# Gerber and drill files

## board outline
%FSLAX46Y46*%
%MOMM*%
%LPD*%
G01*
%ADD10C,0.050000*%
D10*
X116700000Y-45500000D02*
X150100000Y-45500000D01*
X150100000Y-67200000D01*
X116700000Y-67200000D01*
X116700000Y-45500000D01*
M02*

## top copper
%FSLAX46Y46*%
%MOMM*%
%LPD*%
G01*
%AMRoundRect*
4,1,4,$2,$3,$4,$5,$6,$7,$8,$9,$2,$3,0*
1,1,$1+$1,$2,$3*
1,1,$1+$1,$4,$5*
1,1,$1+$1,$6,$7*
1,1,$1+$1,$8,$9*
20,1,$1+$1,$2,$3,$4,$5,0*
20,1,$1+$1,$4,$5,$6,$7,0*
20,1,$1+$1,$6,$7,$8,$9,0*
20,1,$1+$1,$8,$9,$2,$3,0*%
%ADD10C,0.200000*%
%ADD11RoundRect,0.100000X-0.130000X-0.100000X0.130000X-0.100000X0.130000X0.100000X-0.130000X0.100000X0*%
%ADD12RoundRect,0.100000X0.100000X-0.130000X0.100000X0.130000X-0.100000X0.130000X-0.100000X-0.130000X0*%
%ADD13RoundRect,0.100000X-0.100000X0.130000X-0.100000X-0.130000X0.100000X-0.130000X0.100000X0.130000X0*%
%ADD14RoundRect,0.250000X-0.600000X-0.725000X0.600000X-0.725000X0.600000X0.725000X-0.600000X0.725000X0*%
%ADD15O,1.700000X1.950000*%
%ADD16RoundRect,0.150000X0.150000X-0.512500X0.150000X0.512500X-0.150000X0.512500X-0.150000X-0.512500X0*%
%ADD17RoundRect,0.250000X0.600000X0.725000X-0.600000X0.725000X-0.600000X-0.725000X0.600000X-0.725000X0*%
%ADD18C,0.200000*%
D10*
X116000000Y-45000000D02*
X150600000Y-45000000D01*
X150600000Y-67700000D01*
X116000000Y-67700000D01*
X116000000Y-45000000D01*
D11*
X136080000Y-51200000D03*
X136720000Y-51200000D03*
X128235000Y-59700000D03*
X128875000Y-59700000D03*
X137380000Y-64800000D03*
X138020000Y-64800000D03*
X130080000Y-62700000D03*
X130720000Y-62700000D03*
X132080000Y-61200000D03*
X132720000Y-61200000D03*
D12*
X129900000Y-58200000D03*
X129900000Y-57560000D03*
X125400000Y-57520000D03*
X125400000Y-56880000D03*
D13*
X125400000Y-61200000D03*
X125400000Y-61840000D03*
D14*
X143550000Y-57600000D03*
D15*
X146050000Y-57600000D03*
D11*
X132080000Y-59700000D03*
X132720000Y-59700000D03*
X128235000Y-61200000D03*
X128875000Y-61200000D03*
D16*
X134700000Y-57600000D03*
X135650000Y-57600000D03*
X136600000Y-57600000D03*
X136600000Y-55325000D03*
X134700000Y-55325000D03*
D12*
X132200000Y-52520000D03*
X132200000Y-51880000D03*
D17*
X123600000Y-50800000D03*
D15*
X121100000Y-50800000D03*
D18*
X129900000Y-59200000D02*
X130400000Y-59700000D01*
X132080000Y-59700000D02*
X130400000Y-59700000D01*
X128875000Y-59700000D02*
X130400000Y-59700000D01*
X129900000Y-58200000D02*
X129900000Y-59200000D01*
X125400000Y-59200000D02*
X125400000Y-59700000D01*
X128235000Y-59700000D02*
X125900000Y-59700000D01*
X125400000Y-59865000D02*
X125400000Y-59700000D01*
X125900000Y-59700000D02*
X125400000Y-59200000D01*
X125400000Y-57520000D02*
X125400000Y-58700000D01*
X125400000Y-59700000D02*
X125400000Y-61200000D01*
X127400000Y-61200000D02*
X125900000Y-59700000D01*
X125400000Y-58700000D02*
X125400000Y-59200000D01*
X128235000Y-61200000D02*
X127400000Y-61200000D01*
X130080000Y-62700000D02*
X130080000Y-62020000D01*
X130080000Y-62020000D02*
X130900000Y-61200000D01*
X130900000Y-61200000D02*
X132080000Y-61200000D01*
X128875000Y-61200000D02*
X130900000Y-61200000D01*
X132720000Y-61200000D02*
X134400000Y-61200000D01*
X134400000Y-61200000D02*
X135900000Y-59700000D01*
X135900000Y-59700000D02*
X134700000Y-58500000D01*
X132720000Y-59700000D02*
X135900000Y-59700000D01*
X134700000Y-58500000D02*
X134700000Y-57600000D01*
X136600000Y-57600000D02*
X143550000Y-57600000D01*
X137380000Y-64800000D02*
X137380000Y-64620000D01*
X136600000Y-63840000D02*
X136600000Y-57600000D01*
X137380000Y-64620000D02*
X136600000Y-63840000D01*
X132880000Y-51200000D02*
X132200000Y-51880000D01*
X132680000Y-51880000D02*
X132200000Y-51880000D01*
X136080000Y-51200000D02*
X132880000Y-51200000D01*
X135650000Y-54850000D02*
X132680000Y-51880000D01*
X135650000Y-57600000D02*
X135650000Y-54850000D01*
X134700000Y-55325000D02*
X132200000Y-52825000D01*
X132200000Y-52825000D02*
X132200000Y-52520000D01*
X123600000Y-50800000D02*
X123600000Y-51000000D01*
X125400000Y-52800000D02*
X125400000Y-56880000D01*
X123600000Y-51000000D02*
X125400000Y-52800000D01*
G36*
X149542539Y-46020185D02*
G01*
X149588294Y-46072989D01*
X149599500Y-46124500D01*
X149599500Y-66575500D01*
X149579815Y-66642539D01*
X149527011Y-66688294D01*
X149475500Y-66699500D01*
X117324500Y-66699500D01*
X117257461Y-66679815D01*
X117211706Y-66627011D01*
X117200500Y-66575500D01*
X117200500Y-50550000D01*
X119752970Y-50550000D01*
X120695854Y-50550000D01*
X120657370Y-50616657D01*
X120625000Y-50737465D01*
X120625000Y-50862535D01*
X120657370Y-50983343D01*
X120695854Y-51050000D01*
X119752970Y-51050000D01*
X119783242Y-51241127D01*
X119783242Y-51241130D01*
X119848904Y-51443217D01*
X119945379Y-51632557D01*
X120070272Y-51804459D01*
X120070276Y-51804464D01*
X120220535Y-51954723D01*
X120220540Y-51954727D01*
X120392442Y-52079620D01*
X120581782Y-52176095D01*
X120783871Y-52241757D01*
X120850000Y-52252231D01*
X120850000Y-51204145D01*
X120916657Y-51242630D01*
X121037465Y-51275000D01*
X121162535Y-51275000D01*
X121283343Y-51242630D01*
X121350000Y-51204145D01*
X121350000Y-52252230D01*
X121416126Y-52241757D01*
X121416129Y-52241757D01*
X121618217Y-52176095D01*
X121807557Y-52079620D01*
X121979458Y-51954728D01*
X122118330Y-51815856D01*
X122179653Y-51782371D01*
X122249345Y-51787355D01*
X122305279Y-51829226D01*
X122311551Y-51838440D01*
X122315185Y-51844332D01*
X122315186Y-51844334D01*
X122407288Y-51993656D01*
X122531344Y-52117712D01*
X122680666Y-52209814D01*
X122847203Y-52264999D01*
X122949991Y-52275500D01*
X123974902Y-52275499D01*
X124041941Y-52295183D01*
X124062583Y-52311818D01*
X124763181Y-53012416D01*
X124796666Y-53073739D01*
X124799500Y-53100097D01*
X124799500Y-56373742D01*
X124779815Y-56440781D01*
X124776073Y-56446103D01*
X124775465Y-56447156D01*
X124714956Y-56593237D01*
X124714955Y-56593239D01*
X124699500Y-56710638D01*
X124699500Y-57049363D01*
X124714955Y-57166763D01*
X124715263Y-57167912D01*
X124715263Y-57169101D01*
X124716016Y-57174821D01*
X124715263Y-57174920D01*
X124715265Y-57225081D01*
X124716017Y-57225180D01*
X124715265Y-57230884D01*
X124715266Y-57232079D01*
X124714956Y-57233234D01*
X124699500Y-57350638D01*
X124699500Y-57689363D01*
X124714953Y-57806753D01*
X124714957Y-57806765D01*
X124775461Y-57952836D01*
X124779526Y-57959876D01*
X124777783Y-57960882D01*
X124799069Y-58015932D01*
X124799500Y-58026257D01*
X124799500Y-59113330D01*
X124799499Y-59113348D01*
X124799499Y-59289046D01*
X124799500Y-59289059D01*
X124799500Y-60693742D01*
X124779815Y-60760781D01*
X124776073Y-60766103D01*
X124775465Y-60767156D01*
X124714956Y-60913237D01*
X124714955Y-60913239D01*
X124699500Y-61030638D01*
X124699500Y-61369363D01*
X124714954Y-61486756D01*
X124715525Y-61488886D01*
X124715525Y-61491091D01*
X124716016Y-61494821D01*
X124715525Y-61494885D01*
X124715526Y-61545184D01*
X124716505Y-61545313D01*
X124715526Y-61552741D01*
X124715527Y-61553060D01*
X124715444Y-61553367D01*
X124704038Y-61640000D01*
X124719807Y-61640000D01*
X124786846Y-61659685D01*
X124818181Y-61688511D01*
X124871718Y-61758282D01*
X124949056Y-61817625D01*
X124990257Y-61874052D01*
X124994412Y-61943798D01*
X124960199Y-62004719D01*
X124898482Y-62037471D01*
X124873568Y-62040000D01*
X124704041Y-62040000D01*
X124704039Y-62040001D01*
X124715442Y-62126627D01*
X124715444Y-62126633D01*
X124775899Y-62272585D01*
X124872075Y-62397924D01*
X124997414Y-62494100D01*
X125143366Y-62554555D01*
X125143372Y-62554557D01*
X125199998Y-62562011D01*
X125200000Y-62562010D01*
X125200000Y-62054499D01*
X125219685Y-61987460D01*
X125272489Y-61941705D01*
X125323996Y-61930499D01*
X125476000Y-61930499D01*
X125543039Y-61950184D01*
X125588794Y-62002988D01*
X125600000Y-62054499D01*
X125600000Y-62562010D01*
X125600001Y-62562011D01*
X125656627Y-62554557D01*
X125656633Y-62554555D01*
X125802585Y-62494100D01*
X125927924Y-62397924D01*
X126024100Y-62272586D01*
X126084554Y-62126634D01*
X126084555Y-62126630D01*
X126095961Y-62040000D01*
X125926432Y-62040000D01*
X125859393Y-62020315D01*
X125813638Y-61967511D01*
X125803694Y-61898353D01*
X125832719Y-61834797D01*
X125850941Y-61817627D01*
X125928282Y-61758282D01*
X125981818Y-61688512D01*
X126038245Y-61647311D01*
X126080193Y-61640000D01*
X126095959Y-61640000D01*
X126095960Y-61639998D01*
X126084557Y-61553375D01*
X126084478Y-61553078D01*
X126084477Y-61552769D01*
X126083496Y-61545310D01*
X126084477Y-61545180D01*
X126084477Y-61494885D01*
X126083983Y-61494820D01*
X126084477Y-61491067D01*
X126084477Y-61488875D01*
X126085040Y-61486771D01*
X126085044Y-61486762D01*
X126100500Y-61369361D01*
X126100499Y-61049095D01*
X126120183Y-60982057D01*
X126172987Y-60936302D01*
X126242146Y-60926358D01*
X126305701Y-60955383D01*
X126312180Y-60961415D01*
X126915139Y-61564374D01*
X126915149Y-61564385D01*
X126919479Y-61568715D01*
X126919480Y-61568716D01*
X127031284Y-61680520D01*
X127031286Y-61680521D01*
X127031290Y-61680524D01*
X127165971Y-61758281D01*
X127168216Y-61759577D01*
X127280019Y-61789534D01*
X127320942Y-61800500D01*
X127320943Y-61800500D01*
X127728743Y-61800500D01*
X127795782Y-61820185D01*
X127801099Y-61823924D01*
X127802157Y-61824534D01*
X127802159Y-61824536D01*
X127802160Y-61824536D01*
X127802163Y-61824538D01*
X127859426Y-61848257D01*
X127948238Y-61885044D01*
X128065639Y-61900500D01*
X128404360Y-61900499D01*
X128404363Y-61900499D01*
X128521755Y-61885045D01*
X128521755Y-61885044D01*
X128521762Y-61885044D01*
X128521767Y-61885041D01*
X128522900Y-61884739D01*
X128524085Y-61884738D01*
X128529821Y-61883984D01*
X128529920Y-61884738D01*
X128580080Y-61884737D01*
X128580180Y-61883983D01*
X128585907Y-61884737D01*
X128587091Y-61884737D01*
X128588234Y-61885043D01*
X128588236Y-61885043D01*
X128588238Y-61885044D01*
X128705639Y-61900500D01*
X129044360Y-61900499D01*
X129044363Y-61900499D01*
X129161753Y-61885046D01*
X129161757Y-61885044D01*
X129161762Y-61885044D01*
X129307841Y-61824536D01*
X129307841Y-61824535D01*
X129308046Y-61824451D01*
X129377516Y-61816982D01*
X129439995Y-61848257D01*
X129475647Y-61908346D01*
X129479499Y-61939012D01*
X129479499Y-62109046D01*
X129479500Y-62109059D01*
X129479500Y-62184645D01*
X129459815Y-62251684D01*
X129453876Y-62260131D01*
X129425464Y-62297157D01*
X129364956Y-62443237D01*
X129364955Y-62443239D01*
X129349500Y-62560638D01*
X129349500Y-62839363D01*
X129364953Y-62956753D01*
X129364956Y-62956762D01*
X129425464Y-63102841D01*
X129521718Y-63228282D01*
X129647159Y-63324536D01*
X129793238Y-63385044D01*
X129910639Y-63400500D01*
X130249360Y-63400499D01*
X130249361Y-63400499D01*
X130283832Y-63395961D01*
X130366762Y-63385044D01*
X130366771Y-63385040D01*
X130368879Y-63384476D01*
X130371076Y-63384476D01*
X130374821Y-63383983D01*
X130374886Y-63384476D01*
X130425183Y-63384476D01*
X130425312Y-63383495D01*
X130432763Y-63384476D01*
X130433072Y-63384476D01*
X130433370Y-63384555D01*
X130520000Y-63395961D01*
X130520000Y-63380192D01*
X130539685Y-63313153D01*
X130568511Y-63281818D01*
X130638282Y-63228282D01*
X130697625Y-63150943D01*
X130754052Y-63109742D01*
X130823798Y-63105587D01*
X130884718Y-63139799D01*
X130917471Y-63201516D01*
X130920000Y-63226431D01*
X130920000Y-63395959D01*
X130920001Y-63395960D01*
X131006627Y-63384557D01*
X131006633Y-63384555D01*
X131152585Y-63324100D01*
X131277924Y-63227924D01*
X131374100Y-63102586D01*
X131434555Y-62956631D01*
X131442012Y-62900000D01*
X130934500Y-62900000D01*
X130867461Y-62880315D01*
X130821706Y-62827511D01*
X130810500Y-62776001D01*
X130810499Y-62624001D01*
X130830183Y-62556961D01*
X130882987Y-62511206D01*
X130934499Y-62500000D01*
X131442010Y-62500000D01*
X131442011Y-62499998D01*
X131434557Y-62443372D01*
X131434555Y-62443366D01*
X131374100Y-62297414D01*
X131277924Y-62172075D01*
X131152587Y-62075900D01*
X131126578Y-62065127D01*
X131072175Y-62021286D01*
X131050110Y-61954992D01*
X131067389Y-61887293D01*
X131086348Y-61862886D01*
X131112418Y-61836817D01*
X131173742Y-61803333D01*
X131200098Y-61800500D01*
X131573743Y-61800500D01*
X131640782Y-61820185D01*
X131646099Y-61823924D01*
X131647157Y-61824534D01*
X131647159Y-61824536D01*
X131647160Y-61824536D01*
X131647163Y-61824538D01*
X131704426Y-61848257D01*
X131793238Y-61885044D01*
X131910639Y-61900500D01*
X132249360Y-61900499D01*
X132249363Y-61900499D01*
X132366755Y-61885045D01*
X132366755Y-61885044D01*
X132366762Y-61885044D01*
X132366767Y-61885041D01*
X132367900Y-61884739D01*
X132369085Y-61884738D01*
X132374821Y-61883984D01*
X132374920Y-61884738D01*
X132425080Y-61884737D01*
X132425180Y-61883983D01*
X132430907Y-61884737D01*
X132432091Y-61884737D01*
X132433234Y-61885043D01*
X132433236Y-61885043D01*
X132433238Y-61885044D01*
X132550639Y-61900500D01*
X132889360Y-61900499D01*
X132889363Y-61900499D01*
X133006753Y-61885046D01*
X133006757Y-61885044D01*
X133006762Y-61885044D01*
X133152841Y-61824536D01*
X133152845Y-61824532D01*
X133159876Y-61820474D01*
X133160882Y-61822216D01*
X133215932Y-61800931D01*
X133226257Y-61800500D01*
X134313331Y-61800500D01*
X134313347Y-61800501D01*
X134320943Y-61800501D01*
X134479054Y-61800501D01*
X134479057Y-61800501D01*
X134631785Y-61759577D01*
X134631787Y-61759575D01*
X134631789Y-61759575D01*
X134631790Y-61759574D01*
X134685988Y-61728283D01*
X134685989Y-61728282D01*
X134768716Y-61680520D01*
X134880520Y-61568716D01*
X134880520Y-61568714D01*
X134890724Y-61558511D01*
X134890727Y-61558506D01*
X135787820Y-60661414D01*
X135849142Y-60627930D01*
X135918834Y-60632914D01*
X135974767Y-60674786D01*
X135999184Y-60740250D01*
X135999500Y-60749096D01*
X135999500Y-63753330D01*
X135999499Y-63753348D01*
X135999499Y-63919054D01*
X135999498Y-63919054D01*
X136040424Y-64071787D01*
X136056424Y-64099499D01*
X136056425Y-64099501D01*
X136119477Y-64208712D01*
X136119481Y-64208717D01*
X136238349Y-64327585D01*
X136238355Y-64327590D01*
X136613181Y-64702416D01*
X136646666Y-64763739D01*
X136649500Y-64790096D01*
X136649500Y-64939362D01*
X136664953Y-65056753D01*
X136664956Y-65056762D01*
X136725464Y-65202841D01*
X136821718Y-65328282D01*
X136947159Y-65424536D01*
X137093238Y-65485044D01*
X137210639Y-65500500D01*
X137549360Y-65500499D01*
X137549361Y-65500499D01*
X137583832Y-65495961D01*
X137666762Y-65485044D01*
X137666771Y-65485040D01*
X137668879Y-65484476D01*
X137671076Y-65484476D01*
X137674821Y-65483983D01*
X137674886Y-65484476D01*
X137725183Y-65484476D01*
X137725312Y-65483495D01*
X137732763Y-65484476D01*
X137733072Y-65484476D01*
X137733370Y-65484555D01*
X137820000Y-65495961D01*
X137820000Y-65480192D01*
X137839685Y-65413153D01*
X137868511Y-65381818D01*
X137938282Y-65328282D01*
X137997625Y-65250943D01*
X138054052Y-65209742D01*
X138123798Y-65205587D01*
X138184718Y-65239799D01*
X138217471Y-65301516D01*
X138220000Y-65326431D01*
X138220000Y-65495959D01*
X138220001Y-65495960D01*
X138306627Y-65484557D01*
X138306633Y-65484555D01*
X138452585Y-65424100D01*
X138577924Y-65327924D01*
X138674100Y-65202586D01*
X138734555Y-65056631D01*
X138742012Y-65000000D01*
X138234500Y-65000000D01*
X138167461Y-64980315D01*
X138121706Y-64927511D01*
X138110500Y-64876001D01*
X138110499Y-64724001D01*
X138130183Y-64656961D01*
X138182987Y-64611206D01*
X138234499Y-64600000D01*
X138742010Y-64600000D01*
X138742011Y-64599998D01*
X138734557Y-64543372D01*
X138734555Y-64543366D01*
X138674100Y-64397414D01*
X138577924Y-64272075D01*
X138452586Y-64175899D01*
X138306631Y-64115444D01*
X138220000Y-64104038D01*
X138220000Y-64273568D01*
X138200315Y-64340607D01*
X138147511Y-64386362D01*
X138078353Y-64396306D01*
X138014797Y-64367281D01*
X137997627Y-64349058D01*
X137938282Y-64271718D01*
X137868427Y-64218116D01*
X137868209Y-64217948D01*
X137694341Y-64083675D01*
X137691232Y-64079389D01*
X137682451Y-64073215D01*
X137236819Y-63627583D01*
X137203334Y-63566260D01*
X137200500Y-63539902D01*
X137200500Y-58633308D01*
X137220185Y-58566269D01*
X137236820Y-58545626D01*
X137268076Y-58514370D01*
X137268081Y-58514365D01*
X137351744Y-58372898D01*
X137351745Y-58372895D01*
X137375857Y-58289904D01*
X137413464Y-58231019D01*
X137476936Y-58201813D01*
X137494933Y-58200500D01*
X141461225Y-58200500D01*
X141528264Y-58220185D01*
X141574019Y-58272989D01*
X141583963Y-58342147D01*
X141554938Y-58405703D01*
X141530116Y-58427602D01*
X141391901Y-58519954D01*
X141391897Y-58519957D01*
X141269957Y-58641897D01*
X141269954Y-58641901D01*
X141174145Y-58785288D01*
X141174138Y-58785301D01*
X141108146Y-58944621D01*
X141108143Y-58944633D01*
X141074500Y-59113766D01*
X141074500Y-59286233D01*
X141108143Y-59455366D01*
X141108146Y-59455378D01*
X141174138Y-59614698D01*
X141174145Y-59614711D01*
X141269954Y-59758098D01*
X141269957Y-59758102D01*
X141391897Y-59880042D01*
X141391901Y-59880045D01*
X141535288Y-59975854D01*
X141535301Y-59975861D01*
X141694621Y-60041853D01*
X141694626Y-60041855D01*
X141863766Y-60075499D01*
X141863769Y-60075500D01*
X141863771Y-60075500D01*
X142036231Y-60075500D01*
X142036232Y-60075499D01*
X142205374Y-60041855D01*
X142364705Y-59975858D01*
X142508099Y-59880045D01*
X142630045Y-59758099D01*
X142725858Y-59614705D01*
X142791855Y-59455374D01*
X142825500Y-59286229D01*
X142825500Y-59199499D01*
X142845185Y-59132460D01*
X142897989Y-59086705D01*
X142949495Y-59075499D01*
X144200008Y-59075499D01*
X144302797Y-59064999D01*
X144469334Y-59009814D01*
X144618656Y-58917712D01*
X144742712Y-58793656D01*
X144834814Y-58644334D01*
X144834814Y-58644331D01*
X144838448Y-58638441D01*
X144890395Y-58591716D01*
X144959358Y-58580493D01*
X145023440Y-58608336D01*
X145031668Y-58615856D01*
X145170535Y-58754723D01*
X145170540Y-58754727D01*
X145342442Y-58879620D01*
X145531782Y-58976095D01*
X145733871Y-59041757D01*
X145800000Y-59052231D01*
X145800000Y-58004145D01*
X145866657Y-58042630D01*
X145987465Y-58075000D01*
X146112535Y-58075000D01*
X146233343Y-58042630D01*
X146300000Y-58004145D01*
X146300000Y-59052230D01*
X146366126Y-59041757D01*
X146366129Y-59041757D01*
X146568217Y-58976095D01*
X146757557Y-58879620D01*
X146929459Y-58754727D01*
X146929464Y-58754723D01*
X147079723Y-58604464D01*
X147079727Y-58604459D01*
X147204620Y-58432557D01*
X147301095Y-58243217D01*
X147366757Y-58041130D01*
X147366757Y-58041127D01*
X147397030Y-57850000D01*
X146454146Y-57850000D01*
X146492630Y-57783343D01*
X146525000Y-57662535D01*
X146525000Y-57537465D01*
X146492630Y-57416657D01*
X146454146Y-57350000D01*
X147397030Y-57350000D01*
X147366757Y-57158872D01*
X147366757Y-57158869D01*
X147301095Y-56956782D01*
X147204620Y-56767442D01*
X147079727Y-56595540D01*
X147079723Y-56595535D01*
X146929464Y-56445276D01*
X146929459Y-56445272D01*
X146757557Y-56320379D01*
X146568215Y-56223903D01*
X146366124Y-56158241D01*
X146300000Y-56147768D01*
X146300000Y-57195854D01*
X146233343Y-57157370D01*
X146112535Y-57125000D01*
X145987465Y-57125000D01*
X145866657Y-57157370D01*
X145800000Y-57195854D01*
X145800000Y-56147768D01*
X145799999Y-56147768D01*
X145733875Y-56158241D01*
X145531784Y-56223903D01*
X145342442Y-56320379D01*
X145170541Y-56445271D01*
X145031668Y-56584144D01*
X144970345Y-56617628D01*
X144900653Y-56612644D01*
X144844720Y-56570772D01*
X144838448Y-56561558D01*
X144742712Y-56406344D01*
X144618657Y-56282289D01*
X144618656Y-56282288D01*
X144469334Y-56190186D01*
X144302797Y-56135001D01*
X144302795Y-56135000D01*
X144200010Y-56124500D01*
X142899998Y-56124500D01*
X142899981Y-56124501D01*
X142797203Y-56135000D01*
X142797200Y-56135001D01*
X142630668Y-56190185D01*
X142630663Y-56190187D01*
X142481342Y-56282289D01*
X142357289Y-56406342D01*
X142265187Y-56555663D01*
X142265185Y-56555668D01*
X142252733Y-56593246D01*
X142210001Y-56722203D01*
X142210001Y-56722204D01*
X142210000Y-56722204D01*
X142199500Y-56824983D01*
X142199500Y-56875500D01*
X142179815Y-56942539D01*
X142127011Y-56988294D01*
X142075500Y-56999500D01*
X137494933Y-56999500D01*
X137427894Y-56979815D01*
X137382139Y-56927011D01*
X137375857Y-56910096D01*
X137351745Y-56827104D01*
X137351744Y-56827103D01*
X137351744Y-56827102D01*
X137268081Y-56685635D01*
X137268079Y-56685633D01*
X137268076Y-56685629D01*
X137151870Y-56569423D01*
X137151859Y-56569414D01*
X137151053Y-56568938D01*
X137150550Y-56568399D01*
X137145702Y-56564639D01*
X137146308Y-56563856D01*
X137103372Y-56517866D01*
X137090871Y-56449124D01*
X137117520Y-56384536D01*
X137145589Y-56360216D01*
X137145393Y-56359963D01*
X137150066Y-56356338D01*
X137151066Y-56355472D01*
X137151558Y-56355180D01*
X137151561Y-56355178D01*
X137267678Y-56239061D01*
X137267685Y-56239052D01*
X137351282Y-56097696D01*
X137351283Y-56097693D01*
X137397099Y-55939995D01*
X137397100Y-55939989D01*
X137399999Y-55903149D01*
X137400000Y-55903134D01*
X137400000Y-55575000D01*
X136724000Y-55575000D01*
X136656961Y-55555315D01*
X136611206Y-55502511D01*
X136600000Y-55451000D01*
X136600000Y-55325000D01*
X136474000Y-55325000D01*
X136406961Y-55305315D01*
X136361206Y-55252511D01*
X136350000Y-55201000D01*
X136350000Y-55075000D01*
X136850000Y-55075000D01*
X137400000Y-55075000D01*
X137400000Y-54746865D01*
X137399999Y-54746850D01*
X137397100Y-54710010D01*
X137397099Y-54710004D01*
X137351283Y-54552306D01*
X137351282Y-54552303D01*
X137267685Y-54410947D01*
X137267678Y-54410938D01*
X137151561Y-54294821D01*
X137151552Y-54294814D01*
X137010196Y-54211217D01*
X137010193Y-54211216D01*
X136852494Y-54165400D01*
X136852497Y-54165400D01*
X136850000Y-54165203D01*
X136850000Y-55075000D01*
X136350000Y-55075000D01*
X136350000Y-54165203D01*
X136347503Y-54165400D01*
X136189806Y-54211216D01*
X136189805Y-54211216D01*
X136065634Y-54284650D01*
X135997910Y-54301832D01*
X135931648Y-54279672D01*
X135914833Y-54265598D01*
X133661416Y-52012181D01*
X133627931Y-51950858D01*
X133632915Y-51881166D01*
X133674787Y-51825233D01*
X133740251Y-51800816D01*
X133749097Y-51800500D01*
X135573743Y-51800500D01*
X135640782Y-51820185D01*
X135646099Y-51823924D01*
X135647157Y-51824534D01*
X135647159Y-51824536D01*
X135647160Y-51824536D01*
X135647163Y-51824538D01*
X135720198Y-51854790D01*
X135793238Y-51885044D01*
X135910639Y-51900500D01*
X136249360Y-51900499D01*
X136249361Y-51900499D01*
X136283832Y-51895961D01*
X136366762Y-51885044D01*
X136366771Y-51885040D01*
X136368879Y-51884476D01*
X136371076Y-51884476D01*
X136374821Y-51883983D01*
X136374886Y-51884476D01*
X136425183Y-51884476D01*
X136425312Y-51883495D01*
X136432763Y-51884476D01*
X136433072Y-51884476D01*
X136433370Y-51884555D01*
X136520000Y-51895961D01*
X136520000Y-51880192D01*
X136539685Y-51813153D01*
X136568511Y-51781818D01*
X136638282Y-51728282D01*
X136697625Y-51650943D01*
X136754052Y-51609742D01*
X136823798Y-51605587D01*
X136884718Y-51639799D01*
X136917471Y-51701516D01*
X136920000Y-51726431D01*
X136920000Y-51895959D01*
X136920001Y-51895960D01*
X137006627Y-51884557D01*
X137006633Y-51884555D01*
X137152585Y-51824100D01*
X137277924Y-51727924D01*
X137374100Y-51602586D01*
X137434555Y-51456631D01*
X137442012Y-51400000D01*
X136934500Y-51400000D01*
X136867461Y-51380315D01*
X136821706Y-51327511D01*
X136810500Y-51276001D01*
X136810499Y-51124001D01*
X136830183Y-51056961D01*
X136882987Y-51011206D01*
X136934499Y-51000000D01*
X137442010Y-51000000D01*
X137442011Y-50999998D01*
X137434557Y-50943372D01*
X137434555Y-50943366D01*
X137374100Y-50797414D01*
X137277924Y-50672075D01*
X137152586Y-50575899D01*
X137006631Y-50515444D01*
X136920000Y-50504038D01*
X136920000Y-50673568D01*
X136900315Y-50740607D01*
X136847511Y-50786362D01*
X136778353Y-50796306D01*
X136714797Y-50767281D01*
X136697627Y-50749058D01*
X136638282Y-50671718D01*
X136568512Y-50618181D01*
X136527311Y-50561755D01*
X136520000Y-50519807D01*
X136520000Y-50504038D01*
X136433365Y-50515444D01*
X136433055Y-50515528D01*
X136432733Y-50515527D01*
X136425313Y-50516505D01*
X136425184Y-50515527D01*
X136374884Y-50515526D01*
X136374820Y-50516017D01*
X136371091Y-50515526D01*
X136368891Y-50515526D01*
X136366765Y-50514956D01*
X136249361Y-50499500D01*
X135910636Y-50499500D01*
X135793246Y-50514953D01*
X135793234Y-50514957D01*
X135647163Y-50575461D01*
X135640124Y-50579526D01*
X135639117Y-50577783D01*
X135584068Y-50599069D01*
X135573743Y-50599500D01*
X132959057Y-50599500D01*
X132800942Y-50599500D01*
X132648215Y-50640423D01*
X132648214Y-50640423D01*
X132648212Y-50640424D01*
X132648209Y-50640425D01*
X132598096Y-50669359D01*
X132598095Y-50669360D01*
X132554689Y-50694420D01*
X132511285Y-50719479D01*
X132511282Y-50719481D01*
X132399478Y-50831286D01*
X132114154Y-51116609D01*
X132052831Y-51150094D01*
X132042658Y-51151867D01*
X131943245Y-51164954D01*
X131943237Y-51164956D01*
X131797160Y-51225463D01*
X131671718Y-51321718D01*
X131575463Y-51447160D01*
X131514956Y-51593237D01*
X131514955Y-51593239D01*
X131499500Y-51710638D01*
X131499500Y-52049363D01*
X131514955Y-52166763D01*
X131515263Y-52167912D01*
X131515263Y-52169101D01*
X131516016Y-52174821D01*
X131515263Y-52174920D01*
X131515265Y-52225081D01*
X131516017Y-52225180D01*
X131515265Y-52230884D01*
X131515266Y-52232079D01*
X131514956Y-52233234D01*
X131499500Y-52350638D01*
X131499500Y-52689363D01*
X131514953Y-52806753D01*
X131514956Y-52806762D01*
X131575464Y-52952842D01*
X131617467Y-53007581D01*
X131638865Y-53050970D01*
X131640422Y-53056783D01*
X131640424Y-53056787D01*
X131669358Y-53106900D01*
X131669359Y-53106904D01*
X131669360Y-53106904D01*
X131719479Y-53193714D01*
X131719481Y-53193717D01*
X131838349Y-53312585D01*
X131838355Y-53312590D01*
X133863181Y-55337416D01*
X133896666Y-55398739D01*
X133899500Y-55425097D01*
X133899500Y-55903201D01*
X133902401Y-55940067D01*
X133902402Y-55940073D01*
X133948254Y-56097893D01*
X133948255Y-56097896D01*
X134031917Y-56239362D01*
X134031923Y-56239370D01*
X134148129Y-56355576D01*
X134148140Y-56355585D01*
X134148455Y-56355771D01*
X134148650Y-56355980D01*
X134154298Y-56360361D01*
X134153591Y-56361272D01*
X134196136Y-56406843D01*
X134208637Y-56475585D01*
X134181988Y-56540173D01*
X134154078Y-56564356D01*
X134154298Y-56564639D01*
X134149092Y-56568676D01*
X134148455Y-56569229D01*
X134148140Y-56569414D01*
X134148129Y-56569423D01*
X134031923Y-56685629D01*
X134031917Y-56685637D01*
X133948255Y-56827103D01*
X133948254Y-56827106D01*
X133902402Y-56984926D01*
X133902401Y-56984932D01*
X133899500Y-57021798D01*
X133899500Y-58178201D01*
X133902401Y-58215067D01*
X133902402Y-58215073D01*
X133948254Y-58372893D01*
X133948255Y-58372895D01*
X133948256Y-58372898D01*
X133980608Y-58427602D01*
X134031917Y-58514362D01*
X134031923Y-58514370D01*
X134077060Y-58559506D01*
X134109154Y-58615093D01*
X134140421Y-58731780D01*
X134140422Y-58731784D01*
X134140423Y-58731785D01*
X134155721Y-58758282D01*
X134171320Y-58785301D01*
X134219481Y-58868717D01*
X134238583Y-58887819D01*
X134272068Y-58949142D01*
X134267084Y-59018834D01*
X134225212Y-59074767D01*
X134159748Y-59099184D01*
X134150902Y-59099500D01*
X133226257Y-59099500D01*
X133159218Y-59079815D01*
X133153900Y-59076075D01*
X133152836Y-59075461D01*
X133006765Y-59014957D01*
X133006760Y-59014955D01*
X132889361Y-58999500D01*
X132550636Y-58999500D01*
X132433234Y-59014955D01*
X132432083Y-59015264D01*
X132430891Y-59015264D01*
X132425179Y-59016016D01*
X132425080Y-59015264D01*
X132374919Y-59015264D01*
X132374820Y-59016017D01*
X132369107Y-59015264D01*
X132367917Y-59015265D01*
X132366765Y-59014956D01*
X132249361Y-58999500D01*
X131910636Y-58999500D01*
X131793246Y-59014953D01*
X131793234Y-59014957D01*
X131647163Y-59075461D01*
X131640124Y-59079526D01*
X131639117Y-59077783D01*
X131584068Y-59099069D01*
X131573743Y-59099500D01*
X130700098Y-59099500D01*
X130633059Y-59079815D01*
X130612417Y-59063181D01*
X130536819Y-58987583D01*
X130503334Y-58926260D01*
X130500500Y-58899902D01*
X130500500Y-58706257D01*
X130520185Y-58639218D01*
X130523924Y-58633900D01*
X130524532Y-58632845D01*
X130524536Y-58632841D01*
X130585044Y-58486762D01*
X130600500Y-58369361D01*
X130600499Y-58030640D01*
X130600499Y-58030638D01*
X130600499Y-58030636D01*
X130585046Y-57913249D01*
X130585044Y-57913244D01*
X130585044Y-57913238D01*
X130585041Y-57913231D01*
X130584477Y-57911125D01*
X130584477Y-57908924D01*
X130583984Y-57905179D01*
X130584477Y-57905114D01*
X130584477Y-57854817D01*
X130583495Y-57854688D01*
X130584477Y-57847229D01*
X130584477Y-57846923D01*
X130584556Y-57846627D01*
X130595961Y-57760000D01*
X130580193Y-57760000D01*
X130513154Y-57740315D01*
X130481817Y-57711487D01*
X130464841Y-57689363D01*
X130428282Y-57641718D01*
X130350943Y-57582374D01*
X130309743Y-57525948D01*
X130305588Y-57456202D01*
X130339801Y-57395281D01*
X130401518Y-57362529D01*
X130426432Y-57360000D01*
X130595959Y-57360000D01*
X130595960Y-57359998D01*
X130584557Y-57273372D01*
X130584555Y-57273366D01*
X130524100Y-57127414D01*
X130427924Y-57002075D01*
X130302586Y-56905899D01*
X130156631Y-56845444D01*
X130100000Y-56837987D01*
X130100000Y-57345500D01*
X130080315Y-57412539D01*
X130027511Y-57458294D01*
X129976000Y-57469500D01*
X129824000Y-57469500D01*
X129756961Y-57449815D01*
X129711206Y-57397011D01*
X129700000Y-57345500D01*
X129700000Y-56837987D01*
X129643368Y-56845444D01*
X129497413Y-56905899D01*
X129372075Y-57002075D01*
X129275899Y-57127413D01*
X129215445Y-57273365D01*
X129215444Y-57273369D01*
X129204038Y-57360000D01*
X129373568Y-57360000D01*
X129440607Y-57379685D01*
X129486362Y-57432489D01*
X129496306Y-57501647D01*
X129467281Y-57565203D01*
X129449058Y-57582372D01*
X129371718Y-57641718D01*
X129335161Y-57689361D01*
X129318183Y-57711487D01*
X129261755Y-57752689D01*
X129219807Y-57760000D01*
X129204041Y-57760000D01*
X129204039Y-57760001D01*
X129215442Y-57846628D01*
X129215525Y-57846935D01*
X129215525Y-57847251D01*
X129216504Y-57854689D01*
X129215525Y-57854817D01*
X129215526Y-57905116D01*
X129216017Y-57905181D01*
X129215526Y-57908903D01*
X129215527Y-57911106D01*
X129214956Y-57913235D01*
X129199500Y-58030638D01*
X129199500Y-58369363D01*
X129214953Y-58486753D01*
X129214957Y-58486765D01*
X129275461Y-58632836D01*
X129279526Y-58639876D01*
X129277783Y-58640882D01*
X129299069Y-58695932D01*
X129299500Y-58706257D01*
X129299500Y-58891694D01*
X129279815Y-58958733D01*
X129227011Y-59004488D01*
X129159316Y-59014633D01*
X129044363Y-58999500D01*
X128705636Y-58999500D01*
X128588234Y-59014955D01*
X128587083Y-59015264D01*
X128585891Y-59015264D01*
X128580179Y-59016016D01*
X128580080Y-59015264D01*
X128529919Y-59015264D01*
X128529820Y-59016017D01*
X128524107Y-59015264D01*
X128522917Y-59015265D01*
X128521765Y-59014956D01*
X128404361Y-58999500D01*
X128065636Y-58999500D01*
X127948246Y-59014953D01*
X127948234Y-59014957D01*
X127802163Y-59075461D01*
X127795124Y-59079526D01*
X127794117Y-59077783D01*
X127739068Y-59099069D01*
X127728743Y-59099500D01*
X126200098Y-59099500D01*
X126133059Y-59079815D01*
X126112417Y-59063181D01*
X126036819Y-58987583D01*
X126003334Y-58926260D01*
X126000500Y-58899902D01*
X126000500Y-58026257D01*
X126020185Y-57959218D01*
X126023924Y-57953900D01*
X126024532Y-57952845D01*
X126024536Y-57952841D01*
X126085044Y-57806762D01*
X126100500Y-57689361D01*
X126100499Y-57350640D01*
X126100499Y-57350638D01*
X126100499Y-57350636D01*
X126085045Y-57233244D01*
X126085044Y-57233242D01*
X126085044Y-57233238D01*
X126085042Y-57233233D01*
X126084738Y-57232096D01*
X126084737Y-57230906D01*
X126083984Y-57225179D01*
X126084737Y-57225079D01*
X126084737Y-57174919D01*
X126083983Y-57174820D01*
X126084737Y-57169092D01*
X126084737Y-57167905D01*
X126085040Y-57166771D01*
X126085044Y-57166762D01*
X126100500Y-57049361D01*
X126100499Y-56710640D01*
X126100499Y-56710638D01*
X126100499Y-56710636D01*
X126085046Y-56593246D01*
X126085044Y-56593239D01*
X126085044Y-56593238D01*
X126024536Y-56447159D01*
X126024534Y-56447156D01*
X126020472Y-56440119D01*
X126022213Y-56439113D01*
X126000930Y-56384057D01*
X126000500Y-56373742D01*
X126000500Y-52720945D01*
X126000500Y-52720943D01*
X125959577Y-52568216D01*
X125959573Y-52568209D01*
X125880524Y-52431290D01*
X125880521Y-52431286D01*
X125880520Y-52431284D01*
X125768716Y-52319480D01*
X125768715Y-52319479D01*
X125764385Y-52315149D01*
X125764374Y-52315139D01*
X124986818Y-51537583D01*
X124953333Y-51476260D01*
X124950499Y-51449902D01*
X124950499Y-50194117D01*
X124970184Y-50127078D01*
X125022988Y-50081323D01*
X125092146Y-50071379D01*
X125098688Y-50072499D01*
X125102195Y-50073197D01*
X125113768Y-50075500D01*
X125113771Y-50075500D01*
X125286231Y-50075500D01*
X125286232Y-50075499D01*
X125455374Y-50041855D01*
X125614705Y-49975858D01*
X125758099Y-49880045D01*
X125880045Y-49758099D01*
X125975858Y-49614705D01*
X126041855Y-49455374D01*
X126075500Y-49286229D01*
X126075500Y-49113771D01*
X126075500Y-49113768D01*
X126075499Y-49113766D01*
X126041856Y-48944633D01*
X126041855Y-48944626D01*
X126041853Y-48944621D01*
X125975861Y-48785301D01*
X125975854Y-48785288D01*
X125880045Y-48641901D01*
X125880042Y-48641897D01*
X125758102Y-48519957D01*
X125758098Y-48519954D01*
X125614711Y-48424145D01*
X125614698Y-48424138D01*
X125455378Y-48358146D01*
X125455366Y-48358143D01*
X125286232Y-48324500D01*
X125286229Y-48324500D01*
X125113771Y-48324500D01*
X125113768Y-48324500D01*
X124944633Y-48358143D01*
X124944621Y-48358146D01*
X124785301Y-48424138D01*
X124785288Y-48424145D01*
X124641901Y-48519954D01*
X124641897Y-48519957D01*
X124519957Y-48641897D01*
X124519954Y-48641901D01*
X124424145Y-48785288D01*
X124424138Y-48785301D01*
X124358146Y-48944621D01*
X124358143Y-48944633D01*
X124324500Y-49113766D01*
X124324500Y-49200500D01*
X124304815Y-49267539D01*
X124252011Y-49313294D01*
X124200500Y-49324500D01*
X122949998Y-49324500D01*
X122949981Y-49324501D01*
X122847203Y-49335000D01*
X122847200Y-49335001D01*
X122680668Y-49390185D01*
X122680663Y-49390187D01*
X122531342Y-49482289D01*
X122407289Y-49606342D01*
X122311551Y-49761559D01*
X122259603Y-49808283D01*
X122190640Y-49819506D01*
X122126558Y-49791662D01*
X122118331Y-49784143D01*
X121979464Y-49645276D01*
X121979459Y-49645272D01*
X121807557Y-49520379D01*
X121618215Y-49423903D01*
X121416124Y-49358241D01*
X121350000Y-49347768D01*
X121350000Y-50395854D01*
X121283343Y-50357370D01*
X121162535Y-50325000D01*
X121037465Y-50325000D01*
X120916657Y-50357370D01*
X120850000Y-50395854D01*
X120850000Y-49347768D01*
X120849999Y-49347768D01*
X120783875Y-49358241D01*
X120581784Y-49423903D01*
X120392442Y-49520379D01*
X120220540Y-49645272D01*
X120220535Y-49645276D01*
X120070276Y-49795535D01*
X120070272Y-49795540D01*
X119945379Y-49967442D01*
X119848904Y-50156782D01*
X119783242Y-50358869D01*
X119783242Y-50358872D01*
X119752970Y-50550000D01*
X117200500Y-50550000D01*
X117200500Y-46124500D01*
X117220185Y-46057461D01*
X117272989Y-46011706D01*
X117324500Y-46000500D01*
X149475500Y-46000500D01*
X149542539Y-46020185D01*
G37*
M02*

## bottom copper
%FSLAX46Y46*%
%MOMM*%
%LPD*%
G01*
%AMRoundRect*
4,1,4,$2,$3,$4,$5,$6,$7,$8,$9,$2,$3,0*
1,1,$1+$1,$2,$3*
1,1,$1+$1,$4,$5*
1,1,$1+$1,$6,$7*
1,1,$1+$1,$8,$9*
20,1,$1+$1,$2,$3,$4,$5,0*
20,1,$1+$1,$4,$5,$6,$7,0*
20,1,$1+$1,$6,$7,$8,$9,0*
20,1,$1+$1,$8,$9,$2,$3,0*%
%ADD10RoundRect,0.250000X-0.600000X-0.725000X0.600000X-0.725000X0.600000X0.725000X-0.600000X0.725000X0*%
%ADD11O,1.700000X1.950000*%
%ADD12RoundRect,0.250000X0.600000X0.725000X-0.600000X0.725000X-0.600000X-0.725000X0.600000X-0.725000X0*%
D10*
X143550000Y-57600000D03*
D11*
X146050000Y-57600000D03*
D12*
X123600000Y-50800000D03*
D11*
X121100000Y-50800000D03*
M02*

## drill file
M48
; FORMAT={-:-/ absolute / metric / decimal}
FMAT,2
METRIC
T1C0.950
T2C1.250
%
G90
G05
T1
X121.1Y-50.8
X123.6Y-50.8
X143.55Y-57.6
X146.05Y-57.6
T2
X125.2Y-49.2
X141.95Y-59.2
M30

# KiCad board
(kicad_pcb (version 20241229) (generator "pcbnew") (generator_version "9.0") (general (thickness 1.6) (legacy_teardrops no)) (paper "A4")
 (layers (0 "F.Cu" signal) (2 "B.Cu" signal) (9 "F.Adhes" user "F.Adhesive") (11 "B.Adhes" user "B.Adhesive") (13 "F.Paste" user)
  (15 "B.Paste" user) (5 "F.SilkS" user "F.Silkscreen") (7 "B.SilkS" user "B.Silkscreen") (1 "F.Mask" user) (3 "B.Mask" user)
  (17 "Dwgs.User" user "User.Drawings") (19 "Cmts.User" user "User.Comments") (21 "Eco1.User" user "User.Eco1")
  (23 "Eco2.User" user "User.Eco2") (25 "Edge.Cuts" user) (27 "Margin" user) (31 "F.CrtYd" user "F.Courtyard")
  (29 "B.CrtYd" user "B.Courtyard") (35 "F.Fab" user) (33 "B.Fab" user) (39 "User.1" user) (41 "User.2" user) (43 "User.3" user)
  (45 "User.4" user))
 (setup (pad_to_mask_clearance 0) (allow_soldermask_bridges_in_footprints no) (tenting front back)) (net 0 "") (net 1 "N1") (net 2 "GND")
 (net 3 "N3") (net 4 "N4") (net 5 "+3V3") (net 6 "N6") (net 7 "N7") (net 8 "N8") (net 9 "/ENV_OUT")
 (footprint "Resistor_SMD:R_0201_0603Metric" (layer "F.Cu") (at 136.4 51.2)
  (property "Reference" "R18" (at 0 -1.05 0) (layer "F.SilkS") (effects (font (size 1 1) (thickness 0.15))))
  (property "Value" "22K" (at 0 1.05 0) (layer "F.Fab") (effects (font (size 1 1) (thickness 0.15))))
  (pad "" smd roundrect (at -0.345 0) (size 0.318 0.36) (layers "F.Paste") (roundrect_rratio 0.25))
  (pad "" smd roundrect (at 0.345 0) (size 0.318 0.36) (layers "F.Paste") (roundrect_rratio 0.25))
  (pad "1" smd roundrect (at -0.32 0) (size 0.46 0.4) (layers "F.Cu" "F.Mask") (roundrect_rratio 0.25) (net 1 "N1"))
  (pad "2" smd roundrect (at 0.32 0) (size 0.46 0.4) (layers "F.Cu" "F.Mask") (roundrect_rratio 0.25) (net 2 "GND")))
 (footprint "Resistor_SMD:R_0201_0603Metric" (layer "F.Cu") (at 128.555 59.7)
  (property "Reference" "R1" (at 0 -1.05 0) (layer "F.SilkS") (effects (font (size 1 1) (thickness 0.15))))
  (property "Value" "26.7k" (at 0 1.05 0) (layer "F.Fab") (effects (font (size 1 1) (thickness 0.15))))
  (pad "" smd roundrect (at -0.345 0) (size 0.318 0.36) (layers "F.Paste") (roundrect_rratio 0.25))
  (pad "" smd roundrect (at 0.345 0) (size 0.318 0.36) (layers "F.Paste") (roundrect_rratio 0.25))
  (pad "1" smd roundrect (at -0.32 0) (size 0.46 0.4) (layers "F.Cu" "F.Mask") (roundrect_rratio 0.25) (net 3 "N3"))
  (pad "2" smd roundrect (at 0.32 0) (size 0.46 0.4) (layers "F.Cu" "F.Mask") (roundrect_rratio 0.25) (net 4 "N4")))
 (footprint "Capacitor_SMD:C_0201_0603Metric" (layer "F.Cu") (at 137.7 64.8)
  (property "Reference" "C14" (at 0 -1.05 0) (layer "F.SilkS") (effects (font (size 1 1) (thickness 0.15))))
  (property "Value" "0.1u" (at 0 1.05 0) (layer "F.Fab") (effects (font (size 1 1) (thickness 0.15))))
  (pad "" smd roundrect (at -0.345 0) (size 0.318 0.36) (layers "F.Paste") (roundrect_rratio 0.25))
  (pad "" smd roundrect (at 0.345 0) (size 0.318 0.36) (layers "F.Paste") (roundrect_rratio 0.25))
  (pad "1" smd roundrect (at -0.32 0) (size 0.46 0.4) (layers "F.Cu" "F.Mask") (roundrect_rratio 0.25) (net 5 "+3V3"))
  (pad "2" smd roundrect (at 0.32 0) (size 0.46 0.4) (layers "F.Cu" "F.Mask") (roundrect_rratio 0.25) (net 2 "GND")))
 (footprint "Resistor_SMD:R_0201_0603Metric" (layer "F.Cu") (at 130.4 62.7)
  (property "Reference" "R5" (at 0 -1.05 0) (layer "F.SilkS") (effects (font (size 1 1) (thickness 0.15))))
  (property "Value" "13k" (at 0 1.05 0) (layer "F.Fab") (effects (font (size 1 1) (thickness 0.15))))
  (pad "" smd roundrect (at -0.345 0) (size 0.318 0.36) (layers "F.Paste") (roundrect_rratio 0.25))
  (pad "" smd roundrect (at 0.345 0) (size 0.318 0.36) (layers "F.Paste") (roundrect_rratio 0.25))
  (pad "1" smd roundrect (at -0.32 0) (size 0.46 0.4) (layers "F.Cu" "F.Mask") (roundrect_rratio 0.25) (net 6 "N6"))
  (pad "2" smd roundrect (at 0.32 0) (size 0.46 0.4) (layers "F.Cu" "F.Mask") (roundrect_rratio 0.25) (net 2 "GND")))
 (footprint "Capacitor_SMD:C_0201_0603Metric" (layer "F.Cu") (at 132.4 61.2)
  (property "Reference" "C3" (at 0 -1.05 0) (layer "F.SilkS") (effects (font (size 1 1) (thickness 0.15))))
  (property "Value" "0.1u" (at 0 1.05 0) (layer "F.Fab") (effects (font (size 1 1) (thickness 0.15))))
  (pad "" smd roundrect (at -0.345 0) (size 0.318 0.36) (layers "F.Paste") (roundrect_rratio 0.25))
  (pad "" smd roundrect (at 0.345 0) (size 0.318 0.36) (layers "F.Paste") (roundrect_rratio 0.25))
  (pad "1" smd roundrect (at -0.32 0) (size 0.46 0.4) (layers "F.Cu" "F.Mask") (roundrect_rratio 0.25) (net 6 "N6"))
  (pad "2" smd roundrect (at 0.32 0) (size 0.46 0.4) (layers "F.Cu" "F.Mask") (roundrect_rratio 0.25) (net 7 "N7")))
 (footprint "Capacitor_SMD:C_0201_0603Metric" (layer "F.Cu") (at 129.9 57.88 90)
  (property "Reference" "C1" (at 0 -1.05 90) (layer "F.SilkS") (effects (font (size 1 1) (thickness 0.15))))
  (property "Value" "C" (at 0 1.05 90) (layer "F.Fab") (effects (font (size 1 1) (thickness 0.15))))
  (pad "" smd roundrect (at -0.345 0 90) (size 0.318 0.36) (layers "F.Paste") (roundrect_rratio 0.25))
  (pad "" smd roundrect (at 0.345 0 90) (size 0.318 0.36) (layers "F.Paste") (roundrect_rratio 0.25))
  (pad "1" smd roundrect (at -0.32 0 90) (size 0.46 0.4) (layers "F.Cu" "F.Mask") (roundrect_rratio 0.25) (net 4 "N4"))
  (pad "2" smd roundrect (at 0.32 0 90) (size 0.46 0.4) (layers "F.Cu" "F.Mask") (roundrect_rratio 0.25) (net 2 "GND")))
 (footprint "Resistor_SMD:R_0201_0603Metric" (layer "F.Cu") (at 125.4 57.2 90)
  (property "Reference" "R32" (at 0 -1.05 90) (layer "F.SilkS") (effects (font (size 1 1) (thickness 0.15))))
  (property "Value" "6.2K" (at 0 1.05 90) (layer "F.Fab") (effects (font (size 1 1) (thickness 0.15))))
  (pad "" smd roundrect (at -0.345 0 90) (size 0.318 0.36) (layers "F.Paste") (roundrect_rratio 0.25))
  (pad "" smd roundrect (at 0.345 0 90) (size 0.318 0.36) (layers "F.Paste") (roundrect_rratio 0.25))
  (pad "1" smd roundrect (at -0.32 0 90) (size 0.46 0.4) (layers "F.Cu" "F.Mask") (roundrect_rratio 0.25) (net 3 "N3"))
  (pad "2" smd roundrect (at 0.32 0 90) (size 0.46 0.4) (layers "F.Cu" "F.Mask") (roundrect_rratio 0.25) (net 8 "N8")))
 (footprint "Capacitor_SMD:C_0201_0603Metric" (layer "F.Cu") (at 125.4 61.52 -90)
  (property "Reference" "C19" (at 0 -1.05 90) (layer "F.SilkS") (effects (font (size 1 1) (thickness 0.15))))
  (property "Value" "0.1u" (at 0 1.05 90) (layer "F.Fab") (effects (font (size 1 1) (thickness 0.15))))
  (pad "" smd roundrect (at -0.345 0 270) (size 0.318 0.36) (layers "F.Paste") (roundrect_rratio 0.25))
  (pad "" smd roundrect (at 0.345 0 270) (size 0.318 0.36) (layers "F.Paste") (roundrect_rratio 0.25))
  (pad "1" smd roundrect (at -0.32 0 270) (size 0.46 0.4) (layers "F.Cu" "F.Mask") (roundrect_rratio 0.25) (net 3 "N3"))
  (pad "2" smd roundrect (at 0.32 0 270) (size 0.46 0.4) (layers "F.Cu" "F.Mask") (roundrect_rratio 0.25) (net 2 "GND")))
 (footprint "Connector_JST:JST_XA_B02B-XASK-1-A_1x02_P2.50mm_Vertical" (layer "F.Cu") (at 143.55 57.6)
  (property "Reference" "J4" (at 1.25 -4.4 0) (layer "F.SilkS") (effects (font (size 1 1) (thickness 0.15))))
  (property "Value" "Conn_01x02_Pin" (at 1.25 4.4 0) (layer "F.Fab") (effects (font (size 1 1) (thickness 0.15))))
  (pad "" np_thru_hole circle (at -1.6 1.6) (size 1.25 1.25) (drill 1.25) (layers "*.Cu" "*.Mask"))
  (pad "1" thru_hole roundrect (at 0 0) (size 1.7 1.95) (drill 0.95) (layers "*.Cu" "*.Mask") (remove_unused_layers no)
   (roundrect_rratio 0.147059) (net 5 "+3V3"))
  (pad "2" thru_hole oval (at 2.5 0) (size 1.7 1.95) (drill 0.95) (layers "*.Cu" "*.Mask") (remove_unused_layers no) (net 2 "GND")))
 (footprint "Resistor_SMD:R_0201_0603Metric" (layer "F.Cu") (at 132.4 59.7)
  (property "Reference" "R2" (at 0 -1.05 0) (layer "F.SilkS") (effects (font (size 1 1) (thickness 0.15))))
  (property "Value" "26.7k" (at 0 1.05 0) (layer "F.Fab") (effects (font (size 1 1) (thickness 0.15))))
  (pad "" smd roundrect (at -0.345 0) (size 0.318 0.36) (layers "F.Paste") (roundrect_rratio 0.25))
  (pad "" smd roundrect (at 0.345 0) (size 0.318 0.36) (layers "F.Paste") (roundrect_rratio 0.25))
  (pad "1" smd roundrect (at -0.32 0) (size 0.46 0.4) (layers "F.Cu" "F.Mask") (roundrect_rratio 0.25) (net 4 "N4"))
  (pad "2" smd roundrect (at 0.32 0) (size 0.46 0.4) (layers "F.Cu" "F.Mask") (roundrect_rratio 0.25) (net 7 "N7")))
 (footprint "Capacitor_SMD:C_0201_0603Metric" (layer "F.Cu") (at 128.555 61.2)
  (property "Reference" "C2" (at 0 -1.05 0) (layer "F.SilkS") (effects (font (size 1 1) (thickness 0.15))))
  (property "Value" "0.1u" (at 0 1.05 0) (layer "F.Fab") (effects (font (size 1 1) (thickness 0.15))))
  (pad "" smd roundrect (at -0.345 0) (size 0.318 0.36) (layers "F.Paste") (roundrect_rratio 0.25))
  (pad "" smd roundrect (at 0.345 0) (size 0.318 0.36) (layers "F.Paste") (roundrect_rratio 0.25))
  (pad "1" smd roundrect (at -0.32 0) (size 0.46 0.4) (layers "F.Cu" "F.Mask") (roundrect_rratio 0.25) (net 3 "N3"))
  (pad "2" smd roundrect (at 0.32 0) (size 0.46 0.4) (layers "F.Cu" "F.Mask") (roundrect_rratio 0.25) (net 6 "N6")))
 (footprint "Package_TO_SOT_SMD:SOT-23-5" (layer "F.Cu") (at 135.65 56.4625 90)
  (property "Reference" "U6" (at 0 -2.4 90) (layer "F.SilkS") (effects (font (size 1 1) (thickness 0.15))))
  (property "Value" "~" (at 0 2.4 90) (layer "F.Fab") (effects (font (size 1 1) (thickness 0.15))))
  (pad "1" smd roundrect (at -1.1375 -0.95 90) (size 1.325 0.6) (layers "F.Cu" "F.Mask" "F.Paste") (roundrect_rratio 0.25) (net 7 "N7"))
  (pad "2" smd roundrect (at -1.1375 0 90) (size 1.325 0.6) (layers "F.Cu" "F.Mask" "F.Paste") (roundrect_rratio 0.25) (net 1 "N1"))
  (pad "3" smd roundrect (at -1.1375 0.95 90) (size 1.325 0.6) (layers "F.Cu" "F.Mask" "F.Paste") (roundrect_rratio 0.25) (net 5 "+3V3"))
  (pad "4" smd roundrect (at 1.1375 0.95 90) (size 1.325 0.6) (layers "F.Cu" "F.Mask" "F.Paste") (roundrect_rratio 0.25) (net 2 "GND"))
  (pad "5" smd roundrect (at 1.1375 -0.95 90) (size 1.325 0.6) (layers "F.Cu" "F.Mask" "F.Paste") (roundrect_rratio 0.25) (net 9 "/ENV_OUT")))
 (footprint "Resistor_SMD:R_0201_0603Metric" (layer "F.Cu") (at 132.2 52.2 90)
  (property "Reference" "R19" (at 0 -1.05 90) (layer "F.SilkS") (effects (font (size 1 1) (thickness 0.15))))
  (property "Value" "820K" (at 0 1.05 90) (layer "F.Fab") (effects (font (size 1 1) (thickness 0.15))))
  (pad "" smd roundrect (at -0.345 0 90) (size 0.318 0.36) (layers "F.Paste") (roundrect_rratio 0.25))
  (pad "" smd roundrect (at 0.345 0 90) (size 0.318 0.36) (layers "F.Paste") (roundrect_rratio 0.25))
  (pad "1" smd roundrect (at -0.32 0 90) (size 0.46 0.4) (layers "F.Cu" "F.Mask") (roundrect_rratio 0.25) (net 9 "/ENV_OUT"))
  (pad "2" smd roundrect (at 0.32 0 90) (size 0.46 0.4) (layers "F.Cu" "F.Mask") (roundrect_rratio 0.25) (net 1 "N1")))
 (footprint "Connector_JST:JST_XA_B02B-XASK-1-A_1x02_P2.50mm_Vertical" (layer "F.Cu") (at 123.6 50.8 180)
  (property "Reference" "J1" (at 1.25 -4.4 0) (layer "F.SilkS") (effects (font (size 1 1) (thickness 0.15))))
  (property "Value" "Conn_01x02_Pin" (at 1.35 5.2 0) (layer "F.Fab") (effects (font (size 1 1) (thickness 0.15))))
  (pad "" np_thru_hole circle (at -1.6 1.6 180) (size 1.25 1.25) (drill 1.25) (layers "*.Cu" "*.Mask"))
  (pad "1" thru_hole roundrect (at 0 0 180) (size 1.7 1.95) (drill 0.95) (layers "*.Cu" "*.Mask") (remove_unused_layers no)
   (roundrect_rratio 0.147059) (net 8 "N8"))
  (pad "2" thru_hole oval (at 2.5 0 180) (size 1.7 1.95) (drill 0.95) (layers "*.Cu" "*.Mask") (remove_unused_layers no) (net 2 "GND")))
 (gr_rect (start 116 45) (end 150.6 67.7) (stroke (width 0.2) (type default)) (fill no) (layer "F.Cu"))
 (gr_rect (start 116.7 45.5) (end 150.1 67.2) (stroke (width 0.05) (type default)) (fill no) (layer "Edge.Cuts"))
 (segment (start 129.9 59.2) (end 130.4 59.7) (width 0.2) (layer "F.Cu") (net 4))
 (segment (start 132.08 59.7) (end 130.4 59.7) (width 0.2) (layer "F.Cu") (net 4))
 (segment (start 128.875 59.7) (end 130.4 59.7) (width 0.2) (layer "F.Cu") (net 4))
 (segment (start 129.9 58.2) (end 129.9 59.2) (width 0.2) (layer "F.Cu") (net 4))
 (segment (start 125.4 59.2) (end 125.4 59.7) (width 0.2) (layer "F.Cu") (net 3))
 (segment (start 128.235 59.7) (end 125.9 59.7) (width 0.2) (layer "F.Cu") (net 3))
 (segment (start 125.4 59.865) (end 125.4 59.7) (width 0.2) (layer "F.Cu") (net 3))
 (segment (start 125.9 59.7) (end 125.4 59.2) (width 0.2) (layer "F.Cu") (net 3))
 (segment (start 125.4 57.52) (end 125.4 58.7) (width 0.2) (layer "F.Cu") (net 3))
 (segment (start 125.4 59.7) (end 125.4 61.2) (width 0.2) (layer "F.Cu") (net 3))
 (segment (start 127.4 61.2) (end 125.9 59.7) (width 0.2) (layer "F.Cu") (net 3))
 (segment (start 125.4 58.7) (end 125.4 59.2) (width 0.2) (layer "F.Cu") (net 3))
 (segment (start 128.235 61.2) (end 127.4 61.2) (width 0.2) (layer "F.Cu") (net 3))
 (segment (start 130.08 62.7) (end 130.08 62.02) (width 0.2) (layer "F.Cu") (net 6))
 (segment (start 130.08 62.02) (end 130.9 61.2) (width 0.2) (layer "F.Cu") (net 6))
 (segment (start 130.9 61.2) (end 132.08 61.2) (width 0.2) (layer "F.Cu") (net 6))
 (segment (start 128.875 61.2) (end 130.9 61.2) (width 0.2) (layer "F.Cu") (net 6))
 (segment (start 132.72 61.2) (end 134.4 61.2) (width 0.2) (layer "F.Cu") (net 7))
 (segment (start 134.4 61.2) (end 135.9 59.7) (width 0.2) (layer "F.Cu") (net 7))
 (segment (start 135.9 59.7) (end 134.7 58.5) (width 0.2) (layer "F.Cu") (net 7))
 (segment (start 132.72 59.7) (end 135.9 59.7) (width 0.2) (layer "F.Cu") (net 7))
 (segment (start 134.7 58.5) (end 134.7 57.6) (width 0.2) (layer "F.Cu") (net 7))
 (segment (start 136.6 57.6) (end 143.55 57.6) (width 0.2) (layer "F.Cu") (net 5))
 (segment (start 137.38 64.8) (end 137.38 64.62) (width 0.2) (layer "F.Cu") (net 5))
 (segment (start 136.6 63.84) (end 136.6 57.6) (width 0.2) (layer "F.Cu") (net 5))
 (segment (start 137.38 64.62) (end 136.6 63.84) (width 0.2) (layer "F.Cu") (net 5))
 (segment (start 132.88 51.2) (end 132.2 51.88) (width 0.2) (layer "F.Cu") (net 1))
 (segment (start 132.68 51.88) (end 132.2 51.88) (width 0.2) (layer "F.Cu") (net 1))
 (segment (start 136.08 51.2) (end 132.88 51.2) (width 0.2) (layer "F.Cu") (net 1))
 (segment (start 135.65 54.85) (end 132.68 51.88) (width 0.2) (layer "F.Cu") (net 1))
 (segment (start 135.65 57.6) (end 135.65 54.85) (width 0.2) (layer "F.Cu") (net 1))
 (segment (start 134.7 55.325) (end 132.2 52.825) (width 0.2) (layer "F.Cu") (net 9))
 (segment (start 132.2 52.825) (end 132.2 52.52) (width 0.2) (layer "F.Cu") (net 9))
 (segment (start 123.6 50.8) (end 123.6 51) (width 0.2) (layer "F.Cu") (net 8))
 (segment (start 125.4 52.8) (end 125.4 56.88) (width 0.2) (layer "F.Cu") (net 8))
 (segment (start 123.6 51) (end 125.4 52.8) (width 0.2) (layer "F.Cu") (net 8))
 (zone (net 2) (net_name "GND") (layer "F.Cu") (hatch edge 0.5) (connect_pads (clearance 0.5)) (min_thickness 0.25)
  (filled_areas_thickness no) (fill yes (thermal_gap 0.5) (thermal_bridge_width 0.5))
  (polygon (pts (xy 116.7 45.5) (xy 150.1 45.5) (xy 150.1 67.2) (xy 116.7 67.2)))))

